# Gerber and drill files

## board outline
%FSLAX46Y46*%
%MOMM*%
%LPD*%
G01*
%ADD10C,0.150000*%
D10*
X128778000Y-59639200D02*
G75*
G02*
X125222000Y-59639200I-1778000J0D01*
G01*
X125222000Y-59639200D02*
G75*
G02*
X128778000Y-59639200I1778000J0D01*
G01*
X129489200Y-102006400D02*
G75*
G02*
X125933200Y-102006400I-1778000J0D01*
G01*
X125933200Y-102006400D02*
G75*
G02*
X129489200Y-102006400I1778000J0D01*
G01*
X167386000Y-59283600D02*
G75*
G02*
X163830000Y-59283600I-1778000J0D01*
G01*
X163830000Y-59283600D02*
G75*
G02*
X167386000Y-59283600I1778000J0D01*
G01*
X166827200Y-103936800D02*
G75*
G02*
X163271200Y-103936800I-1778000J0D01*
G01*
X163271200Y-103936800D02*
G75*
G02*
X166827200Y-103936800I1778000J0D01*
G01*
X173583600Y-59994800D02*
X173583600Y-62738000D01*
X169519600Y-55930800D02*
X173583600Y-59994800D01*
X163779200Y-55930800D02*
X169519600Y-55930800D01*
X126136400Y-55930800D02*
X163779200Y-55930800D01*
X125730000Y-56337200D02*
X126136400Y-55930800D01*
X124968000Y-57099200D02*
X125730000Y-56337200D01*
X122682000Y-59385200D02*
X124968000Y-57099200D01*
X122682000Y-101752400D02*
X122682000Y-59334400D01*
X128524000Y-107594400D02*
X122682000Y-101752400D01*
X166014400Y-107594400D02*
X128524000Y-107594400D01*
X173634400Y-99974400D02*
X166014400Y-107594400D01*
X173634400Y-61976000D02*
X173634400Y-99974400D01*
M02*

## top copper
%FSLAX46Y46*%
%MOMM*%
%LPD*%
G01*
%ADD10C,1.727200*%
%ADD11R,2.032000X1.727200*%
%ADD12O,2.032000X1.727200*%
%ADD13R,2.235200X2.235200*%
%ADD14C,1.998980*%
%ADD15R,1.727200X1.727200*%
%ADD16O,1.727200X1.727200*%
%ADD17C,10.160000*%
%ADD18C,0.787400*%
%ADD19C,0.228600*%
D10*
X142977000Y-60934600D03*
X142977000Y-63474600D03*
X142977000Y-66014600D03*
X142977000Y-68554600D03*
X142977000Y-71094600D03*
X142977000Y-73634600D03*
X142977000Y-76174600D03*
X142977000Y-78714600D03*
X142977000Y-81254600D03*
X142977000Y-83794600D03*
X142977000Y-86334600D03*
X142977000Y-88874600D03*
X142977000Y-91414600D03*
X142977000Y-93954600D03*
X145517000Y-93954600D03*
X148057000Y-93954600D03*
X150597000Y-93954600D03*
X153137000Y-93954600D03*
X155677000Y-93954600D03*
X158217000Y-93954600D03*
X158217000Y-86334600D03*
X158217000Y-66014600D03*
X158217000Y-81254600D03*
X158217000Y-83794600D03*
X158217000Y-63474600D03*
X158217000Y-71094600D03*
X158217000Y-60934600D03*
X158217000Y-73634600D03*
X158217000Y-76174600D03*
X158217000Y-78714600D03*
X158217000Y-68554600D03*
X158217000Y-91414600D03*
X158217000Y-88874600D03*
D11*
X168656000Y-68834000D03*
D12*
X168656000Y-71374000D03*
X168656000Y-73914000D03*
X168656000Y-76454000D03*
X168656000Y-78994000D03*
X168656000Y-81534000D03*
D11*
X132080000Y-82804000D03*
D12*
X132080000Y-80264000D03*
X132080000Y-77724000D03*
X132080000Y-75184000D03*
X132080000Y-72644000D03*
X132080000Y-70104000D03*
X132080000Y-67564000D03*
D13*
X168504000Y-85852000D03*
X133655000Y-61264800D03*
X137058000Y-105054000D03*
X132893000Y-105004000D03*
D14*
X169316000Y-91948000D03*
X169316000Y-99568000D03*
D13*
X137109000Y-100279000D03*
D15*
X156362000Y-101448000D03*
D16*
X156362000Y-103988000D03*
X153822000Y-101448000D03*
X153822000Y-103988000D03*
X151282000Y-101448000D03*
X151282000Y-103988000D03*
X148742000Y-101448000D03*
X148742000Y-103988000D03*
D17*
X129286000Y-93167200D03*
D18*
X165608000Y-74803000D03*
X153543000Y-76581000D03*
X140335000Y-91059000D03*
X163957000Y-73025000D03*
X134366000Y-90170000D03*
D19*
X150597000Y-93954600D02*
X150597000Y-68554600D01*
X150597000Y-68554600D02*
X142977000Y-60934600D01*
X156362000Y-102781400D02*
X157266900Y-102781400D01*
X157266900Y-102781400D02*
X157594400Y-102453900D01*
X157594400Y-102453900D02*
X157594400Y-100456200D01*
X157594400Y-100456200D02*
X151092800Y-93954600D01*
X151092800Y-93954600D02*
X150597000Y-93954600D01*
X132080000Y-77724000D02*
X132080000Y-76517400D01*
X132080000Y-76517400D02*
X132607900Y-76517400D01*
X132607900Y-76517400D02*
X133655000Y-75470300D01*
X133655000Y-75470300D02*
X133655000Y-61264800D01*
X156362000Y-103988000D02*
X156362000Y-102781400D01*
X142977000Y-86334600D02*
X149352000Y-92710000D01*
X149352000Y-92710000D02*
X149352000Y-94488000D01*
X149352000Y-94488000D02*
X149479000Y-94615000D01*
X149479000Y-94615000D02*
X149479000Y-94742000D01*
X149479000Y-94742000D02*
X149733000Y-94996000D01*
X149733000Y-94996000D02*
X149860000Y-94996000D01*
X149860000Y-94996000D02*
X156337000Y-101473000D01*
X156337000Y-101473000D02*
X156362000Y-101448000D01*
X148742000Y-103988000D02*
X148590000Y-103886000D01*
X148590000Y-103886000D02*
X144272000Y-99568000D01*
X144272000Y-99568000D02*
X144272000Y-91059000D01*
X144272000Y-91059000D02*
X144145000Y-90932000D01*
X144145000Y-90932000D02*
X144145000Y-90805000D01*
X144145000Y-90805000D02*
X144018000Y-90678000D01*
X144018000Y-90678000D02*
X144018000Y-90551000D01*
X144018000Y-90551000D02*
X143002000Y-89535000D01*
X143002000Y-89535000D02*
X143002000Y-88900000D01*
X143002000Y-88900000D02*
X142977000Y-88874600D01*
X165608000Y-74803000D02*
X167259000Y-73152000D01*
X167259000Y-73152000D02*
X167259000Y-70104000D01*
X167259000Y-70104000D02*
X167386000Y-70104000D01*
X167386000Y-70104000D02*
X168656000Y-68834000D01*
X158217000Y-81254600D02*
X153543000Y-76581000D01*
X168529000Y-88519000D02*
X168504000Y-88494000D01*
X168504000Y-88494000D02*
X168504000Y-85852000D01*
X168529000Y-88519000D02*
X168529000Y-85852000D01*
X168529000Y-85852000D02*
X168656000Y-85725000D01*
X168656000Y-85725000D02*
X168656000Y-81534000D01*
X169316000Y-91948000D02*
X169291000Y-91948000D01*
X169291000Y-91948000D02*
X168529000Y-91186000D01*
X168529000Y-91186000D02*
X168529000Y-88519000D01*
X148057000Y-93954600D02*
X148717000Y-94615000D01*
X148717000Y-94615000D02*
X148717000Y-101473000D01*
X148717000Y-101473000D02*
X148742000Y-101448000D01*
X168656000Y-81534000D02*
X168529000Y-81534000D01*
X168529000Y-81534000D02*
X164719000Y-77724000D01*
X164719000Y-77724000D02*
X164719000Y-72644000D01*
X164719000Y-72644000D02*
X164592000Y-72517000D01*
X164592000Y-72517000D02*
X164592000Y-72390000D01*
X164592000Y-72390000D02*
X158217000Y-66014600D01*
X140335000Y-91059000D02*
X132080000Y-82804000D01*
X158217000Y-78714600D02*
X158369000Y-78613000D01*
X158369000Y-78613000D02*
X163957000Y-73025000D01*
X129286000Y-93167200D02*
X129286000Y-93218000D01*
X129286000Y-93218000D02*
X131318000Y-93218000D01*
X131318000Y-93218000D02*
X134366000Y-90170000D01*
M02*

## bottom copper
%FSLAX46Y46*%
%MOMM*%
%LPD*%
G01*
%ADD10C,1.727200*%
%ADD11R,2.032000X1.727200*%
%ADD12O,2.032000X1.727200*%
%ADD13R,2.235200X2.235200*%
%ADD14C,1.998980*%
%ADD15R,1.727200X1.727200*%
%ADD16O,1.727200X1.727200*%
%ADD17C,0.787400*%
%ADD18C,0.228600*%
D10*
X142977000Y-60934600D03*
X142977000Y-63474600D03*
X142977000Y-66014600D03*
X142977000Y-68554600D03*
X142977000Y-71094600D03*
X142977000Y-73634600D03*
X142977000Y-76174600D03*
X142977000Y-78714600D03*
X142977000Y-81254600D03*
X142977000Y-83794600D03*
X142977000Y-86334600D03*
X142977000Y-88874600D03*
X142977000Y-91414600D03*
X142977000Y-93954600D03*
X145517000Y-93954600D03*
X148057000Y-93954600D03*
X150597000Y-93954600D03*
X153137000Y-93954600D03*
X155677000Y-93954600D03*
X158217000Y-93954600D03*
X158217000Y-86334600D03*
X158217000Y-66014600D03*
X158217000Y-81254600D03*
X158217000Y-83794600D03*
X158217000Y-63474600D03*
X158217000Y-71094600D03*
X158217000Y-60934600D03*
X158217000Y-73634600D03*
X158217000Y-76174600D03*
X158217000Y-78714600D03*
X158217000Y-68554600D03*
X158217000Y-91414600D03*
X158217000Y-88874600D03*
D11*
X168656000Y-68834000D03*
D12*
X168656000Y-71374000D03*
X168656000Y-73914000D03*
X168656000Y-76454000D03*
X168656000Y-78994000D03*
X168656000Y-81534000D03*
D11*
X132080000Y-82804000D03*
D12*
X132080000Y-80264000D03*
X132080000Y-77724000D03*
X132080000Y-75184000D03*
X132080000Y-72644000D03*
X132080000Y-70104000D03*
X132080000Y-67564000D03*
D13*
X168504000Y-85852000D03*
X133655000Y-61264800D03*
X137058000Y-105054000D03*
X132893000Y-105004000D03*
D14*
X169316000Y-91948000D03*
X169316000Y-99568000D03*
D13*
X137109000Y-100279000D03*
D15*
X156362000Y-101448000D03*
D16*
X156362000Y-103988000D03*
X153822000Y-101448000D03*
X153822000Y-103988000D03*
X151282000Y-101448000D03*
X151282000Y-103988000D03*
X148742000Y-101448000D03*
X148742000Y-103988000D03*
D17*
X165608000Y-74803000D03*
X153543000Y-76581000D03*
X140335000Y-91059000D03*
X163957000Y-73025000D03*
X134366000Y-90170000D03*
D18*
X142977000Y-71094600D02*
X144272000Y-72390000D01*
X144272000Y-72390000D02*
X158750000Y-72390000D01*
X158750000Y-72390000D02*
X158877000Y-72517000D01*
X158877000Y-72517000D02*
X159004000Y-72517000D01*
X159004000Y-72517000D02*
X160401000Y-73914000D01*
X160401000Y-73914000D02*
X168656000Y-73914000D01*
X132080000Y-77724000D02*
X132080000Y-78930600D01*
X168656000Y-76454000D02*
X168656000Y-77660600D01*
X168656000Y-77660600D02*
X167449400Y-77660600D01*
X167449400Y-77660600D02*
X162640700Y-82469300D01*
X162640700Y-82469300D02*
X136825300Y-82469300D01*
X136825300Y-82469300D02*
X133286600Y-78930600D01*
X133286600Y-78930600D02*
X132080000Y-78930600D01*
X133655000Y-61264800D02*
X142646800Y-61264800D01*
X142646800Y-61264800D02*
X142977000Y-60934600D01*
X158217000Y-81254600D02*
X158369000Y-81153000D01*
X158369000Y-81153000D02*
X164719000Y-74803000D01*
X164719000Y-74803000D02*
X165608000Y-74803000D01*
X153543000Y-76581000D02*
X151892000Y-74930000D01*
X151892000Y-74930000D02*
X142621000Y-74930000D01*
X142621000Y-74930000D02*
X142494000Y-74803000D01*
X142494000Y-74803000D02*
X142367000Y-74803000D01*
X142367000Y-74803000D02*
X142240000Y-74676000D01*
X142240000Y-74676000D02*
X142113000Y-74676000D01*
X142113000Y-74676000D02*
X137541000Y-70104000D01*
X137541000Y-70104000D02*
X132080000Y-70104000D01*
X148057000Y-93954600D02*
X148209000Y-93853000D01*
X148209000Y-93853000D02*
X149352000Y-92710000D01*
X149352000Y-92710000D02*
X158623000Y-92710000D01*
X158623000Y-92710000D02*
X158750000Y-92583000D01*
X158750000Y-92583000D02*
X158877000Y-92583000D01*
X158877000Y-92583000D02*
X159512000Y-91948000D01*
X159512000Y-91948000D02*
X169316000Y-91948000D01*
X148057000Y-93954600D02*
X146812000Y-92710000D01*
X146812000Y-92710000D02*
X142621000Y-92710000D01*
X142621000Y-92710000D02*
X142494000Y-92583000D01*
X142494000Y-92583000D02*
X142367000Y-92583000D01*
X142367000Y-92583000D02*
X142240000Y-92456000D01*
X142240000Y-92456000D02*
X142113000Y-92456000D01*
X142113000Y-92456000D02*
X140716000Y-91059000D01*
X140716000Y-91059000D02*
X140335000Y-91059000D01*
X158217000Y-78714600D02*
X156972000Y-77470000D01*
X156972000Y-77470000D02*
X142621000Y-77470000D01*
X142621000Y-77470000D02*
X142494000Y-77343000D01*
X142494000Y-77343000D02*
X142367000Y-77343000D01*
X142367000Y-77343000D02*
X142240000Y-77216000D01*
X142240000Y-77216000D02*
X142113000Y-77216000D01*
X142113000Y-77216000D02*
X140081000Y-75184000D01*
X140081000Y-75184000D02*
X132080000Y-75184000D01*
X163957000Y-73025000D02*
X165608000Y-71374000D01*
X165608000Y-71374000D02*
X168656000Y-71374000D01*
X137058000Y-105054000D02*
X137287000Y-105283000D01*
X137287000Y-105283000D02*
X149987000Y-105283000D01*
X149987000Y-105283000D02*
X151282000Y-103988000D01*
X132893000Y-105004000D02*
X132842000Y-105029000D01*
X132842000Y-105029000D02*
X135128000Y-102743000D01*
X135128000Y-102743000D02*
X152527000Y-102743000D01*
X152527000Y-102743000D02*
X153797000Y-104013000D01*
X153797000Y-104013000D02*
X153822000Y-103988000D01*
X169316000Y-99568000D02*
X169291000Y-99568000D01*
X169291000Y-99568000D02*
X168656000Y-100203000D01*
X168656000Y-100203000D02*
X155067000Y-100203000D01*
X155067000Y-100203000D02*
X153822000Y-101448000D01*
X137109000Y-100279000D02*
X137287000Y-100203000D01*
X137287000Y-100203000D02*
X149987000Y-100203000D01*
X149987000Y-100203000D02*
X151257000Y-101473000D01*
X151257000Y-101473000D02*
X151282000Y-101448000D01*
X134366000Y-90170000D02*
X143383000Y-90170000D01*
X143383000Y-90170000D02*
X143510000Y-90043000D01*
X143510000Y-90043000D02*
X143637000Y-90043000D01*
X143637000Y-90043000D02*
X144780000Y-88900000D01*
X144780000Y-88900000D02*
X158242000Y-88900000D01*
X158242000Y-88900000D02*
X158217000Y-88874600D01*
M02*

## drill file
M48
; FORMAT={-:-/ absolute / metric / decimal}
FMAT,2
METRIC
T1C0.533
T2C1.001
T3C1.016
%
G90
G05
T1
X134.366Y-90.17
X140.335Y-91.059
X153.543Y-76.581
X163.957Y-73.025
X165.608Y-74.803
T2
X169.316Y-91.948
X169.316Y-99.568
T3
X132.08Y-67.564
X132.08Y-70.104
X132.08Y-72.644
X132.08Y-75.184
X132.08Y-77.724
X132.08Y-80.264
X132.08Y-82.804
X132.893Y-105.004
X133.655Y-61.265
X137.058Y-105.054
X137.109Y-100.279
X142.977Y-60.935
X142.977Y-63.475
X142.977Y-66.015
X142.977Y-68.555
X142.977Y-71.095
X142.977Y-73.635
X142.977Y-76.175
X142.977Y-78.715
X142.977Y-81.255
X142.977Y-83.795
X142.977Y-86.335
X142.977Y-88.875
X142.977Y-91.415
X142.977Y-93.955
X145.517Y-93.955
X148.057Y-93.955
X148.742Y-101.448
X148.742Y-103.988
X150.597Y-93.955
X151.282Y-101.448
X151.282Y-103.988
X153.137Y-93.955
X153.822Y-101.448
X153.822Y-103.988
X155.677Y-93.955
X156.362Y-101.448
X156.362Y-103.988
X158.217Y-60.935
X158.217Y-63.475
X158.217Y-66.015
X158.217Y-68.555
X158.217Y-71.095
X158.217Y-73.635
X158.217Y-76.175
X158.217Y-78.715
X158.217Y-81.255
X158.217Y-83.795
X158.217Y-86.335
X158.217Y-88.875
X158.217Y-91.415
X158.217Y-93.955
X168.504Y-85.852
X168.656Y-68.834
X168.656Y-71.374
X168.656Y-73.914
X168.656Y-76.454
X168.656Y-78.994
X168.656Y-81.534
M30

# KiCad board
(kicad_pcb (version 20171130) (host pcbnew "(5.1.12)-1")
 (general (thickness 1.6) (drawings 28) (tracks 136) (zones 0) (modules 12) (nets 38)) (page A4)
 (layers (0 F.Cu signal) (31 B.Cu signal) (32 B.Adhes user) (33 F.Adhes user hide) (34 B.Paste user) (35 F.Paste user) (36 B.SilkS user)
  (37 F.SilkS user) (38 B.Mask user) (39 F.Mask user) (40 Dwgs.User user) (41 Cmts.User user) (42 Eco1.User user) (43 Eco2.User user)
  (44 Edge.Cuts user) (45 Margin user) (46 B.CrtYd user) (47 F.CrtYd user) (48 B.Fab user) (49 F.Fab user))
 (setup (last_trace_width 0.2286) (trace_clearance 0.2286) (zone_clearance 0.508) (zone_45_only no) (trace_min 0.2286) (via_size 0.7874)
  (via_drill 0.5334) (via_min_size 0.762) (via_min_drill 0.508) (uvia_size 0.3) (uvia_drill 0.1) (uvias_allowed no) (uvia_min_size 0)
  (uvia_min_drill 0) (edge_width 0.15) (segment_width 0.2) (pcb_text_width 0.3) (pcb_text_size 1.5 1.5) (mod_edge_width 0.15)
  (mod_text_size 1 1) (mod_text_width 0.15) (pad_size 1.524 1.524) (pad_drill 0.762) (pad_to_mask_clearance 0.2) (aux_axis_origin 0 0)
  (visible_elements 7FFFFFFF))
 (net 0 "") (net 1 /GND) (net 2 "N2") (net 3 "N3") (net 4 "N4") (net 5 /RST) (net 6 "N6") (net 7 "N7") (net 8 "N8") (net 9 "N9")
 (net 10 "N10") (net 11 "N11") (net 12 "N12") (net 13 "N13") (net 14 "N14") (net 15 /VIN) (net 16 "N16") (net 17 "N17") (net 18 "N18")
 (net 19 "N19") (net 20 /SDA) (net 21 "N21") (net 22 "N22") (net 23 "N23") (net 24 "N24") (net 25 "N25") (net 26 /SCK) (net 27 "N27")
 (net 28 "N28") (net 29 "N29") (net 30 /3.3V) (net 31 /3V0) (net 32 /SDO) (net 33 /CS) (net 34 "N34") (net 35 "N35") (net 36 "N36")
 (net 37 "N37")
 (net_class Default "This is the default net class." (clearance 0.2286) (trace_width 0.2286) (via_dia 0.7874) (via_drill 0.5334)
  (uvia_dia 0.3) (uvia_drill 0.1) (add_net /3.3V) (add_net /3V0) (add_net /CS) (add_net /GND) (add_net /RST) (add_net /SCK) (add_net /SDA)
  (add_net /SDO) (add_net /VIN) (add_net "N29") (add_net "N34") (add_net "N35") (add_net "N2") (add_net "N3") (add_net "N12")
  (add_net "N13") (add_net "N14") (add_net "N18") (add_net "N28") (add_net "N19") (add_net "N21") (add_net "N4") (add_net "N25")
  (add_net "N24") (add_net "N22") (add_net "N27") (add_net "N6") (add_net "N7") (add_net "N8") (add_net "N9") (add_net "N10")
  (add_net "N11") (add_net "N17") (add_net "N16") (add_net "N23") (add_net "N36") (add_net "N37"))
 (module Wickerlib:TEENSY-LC (layer F.Cu) (at 153.137 71.0946)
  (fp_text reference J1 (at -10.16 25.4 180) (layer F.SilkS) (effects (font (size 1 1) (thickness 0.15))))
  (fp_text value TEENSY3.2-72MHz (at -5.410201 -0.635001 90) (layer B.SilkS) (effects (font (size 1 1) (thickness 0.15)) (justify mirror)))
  (pad G1 thru_hole circle (at -10.16 -10.16) (size 1.7272 1.7272) (drill 1.016) (layers *.Cu *.Mask F.SilkS) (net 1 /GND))
  (pad 0 thru_hole circle (at -10.16 -7.62) (size 1.7272 1.7272) (drill 1.016) (layers *.Cu *.Mask F.SilkS) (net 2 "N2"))
  (pad 1 thru_hole circle (at -10.16 -5.08) (size 1.7272 1.7272) (drill 1.016) (layers *.Cu *.Mask F.SilkS) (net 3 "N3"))
  (pad 2 thru_hole circle (at -10.16 -2.54) (size 1.7272 1.7272) (drill 1.016) (layers *.Cu *.Mask F.SilkS) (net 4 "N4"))
  (pad 3 thru_hole circle (at -10.16 0) (size 1.7272 1.7272) (drill 1.016) (layers *.Cu *.Mask F.SilkS) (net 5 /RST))
  (pad 4 thru_hole circle (at -10.16 2.54) (size 1.7272 1.7272) (drill 1.016) (layers *.Cu *.Mask F.SilkS) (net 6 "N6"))
  (pad 5 thru_hole circle (at -10.16 5.08) (size 1.7272 1.7272) (drill 1.016) (layers *.Cu *.Mask F.SilkS) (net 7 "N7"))
  (pad 6 thru_hole circle (at -10.16 7.62) (size 1.7272 1.7272) (drill 1.016) (layers *.Cu *.Mask F.SilkS) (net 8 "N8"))
  (pad 7 thru_hole circle (at -10.16 10.16) (size 1.7272 1.7272) (drill 1.016) (layers *.Cu *.Mask F.SilkS) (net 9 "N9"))
  (pad 8 thru_hole circle (at -10.16 12.7) (size 1.7272 1.7272) (drill 1.016) (layers *.Cu *.Mask F.SilkS) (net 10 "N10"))
  (pad 9 thru_hole circle (at -10.16 15.24) (size 1.7272 1.7272) (drill 1.016) (layers *.Cu *.Mask F.SilkS) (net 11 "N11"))
  (pad 10 thru_hole circle (at -10.16 17.78) (size 1.7272 1.7272) (drill 1.016) (layers *.Cu *.Mask F.SilkS) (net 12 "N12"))
  (pad 11 thru_hole circle (at -10.16 20.32) (size 1.7272 1.7272) (drill 1.016) (layers *.Cu *.Mask F.SilkS) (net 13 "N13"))
  (pad 12 thru_hole circle (at -10.16 22.86) (size 1.7272 1.7272) (drill 1.016) (layers *.Cu *.Mask F.SilkS) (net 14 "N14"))
  (pad 17A thru_hole circle (at -7.62 22.86) (size 1.7272 1.7272) (drill 1.016) (layers *.Cu *.Mask F.SilkS))
  (pad 3V1 thru_hole circle (at -5.08 22.86) (size 1.7272 1.7272) (drill 1.016) (layers *.Cu *.Mask F.SilkS) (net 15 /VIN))
  (pad G2 thru_hole circle (at -2.54 22.86) (size 1.7272 1.7272) (drill 1.016) (layers *.Cu *.Mask F.SilkS) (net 1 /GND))
  (pad PGM thru_hole circle (at 0 22.86) (size 1.7272 1.7272) (drill 1.016) (layers *.Cu *.Mask F.SilkS) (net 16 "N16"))
  (pad DAC thru_hole circle (at 2.54 22.86) (size 1.7272 1.7272) (drill 1.016) (layers *.Cu *.Mask F.SilkS) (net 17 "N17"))
  (pad 13 thru_hole circle (at 5.08 22.86) (size 1.7272 1.7272) (drill 1.016) (layers *.Cu *.Mask F.SilkS) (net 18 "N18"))
  (pad 16 thru_hole circle (at 5.08 15.24) (size 1.7272 1.7272) (drill 1.016) (layers *.Cu *.Mask F.SilkS) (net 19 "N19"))
  (pad 3V2 thru_hole circle (at 5.08 -5.08) (size 1.7272 1.7272) (drill 1.016) (layers *.Cu *.Mask F.SilkS) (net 15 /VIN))
  (pad 18 thru_hole circle (at 5.08 10.16) (size 1.7272 1.7272) (drill 1.016) (layers *.Cu *.Mask F.SilkS) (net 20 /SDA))
  (pad 17 thru_hole circle (at 5.08 12.7) (size 1.7272 1.7272) (drill 1.016) (layers *.Cu *.Mask F.SilkS) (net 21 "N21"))
  (pad G3 thru_hole circle (at 5.08 -7.62) (size 1.7272 1.7272) (drill 1.016) (layers *.Cu *.Mask F.SilkS))
  (pad 22 thru_hole circle (at 5.08 0) (size 1.7272 1.7272) (drill 1.016) (layers *.Cu *.Mask F.SilkS) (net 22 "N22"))
  (pad VIN thru_hole circle (at 5.08 -10.16) (size 1.7272 1.7272) (drill 1.016) (layers *.Cu *.Mask F.SilkS) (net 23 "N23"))
  (pad 21 thru_hole circle (at 5.08 2.54) (size 1.7272 1.7272) (drill 1.016) (layers *.Cu *.Mask F.SilkS) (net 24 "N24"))
  (pad 20 thru_hole circle (at 5.08 5.08) (size 1.7272 1.7272) (drill 1.016) (layers *.Cu *.Mask F.SilkS) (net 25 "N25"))
  (pad 19 thru_hole circle (at 5.08 7.62) (size 1.7272 1.7272) (drill 1.016) (layers *.Cu *.Mask F.SilkS) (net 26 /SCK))
  (pad 23 thru_hole circle (at 5.08 -2.54) (size 1.7272 1.7272) (drill 1.016) (layers *.Cu *.Mask F.SilkS) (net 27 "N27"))
  (pad 14 thru_hole circle (at 5.08 20.32) (size 1.7272 1.7272) (drill 1.016) (layers *.Cu *.Mask F.SilkS) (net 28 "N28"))
  (pad 15 thru_hole circle (at 5.08 17.78) (size 1.7272 1.7272) (drill 1.016) (layers *.Cu *.Mask F.SilkS) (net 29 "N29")))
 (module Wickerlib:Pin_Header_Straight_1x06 (layer F.Cu) (at 168.656 68.834)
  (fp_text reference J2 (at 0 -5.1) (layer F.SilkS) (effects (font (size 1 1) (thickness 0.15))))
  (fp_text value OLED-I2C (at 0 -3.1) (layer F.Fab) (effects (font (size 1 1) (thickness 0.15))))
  (pad 1 thru_hole rect (at 0 0) (size 2.032 1.7272) (drill 1.016) (layers *.Cu *.Mask F.SilkS) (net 20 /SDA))
  (pad 2 thru_hole oval (at 0 2.54) (size 2.032 1.7272) (drill 1.016) (layers *.Cu *.Mask F.SilkS) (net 26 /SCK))
  (pad 3 thru_hole oval (at 0 5.08) (size 2.032 1.7272) (drill 1.016) (layers *.Cu *.Mask F.SilkS) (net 5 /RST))
  (pad 4 thru_hole oval (at 0 7.62) (size 2.032 1.7272) (drill 1.016) (layers *.Cu *.Mask F.SilkS) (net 1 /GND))
  (pad 5 thru_hole oval (at 0 10.16) (size 2.032 1.7272) (drill 1.016) (layers *.Cu *.Mask F.SilkS) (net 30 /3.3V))
  (pad 6 thru_hole oval (at 0 12.7) (size 2.032 1.7272) (drill 1.016) (layers *.Cu *.Mask F.SilkS) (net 15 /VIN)))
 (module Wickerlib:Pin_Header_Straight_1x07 (layer F.Cu) (at 132.08 82.804 180)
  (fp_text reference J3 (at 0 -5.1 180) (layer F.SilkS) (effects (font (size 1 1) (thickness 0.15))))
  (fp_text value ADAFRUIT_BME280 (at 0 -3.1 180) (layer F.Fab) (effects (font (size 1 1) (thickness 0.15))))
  (pad 1 thru_hole rect (at 0 0 180) (size 2.032 1.7272) (drill 1.016) (layers *.Cu *.Mask F.SilkS) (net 15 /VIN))
  (pad 2 thru_hole oval (at 0 2.54 180) (size 2.032 1.7272) (drill 1.016) (layers *.Cu *.Mask F.SilkS) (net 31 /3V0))
  (pad 3 thru_hole oval (at 0 5.08 180) (size 2.032 1.7272) (drill 1.016) (layers *.Cu *.Mask F.SilkS) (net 1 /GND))
  (pad 4 thru_hole oval (at 0 7.62 180) (size 2.032 1.7272) (drill 1.016) (layers *.Cu *.Mask F.SilkS) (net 26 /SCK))
  (pad 5 thru_hole oval (at 0 10.16 180) (size 2.032 1.7272) (drill 1.016) (layers *.Cu *.Mask F.SilkS) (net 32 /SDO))
  (pad 6 thru_hole oval (at 0 12.7 180) (size 2.032 1.7272) (drill 1.016) (layers *.Cu *.Mask F.SilkS) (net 20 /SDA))
  (pad 7 thru_hole oval (at 0 15.24 180) (size 2.032 1.7272) (drill 1.016) (layers *.Cu *.Mask F.SilkS) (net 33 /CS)))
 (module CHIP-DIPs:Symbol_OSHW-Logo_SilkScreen (layer F.Cu) (at 129.286 93.0148 270)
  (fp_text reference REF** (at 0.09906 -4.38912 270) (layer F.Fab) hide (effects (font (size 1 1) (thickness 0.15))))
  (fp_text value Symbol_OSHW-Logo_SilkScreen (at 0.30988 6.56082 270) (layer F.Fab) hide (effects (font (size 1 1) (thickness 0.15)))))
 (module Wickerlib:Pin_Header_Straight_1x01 (layer F.Cu) (at 168.504 85.852 90)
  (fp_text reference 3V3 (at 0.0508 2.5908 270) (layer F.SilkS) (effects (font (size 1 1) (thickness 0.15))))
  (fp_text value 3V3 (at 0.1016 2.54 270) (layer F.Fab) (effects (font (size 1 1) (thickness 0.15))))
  (pad 1 thru_hole rect (at 0 0 90) (size 2.2352 2.2352) (drill 1.016) (layers *.Cu *.Mask F.SilkS) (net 15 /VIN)))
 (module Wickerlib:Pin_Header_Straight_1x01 (layer F.Cu) (at 133.655 61.2648)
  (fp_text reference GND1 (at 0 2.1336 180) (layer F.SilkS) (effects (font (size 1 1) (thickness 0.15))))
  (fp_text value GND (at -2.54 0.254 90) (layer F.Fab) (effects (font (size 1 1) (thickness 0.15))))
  (pad 1 thru_hole rect (at 0 0) (size 2.2352 2.2352) (drill 1.016) (layers *.Cu *.Mask F.SilkS) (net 1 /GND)))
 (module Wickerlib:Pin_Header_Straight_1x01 (layer F.Cu) (at 137.058 105.054 270)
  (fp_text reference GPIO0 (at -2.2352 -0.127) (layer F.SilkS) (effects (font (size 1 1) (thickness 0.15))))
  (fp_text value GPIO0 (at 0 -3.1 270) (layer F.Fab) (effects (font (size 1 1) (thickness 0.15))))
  (pad 1 thru_hole rect (at 0 0 270) (size 2.2352 2.2352) (drill 1.016) (layers *.Cu *.Mask F.SilkS) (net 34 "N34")))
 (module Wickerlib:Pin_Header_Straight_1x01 (layer F.Cu) (at 132.893 105.004 270)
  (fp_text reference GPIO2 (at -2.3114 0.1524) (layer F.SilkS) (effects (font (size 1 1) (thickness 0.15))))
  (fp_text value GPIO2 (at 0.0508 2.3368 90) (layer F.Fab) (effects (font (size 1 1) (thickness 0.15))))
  (pad 1 thru_hole rect (at 0 0 270) (size 2.2352 2.2352) (drill 1.016) (layers *.Cu *.Mask F.SilkS) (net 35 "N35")))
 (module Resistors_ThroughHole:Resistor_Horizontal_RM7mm (layer F.Cu) (at 169.316 91.948 270)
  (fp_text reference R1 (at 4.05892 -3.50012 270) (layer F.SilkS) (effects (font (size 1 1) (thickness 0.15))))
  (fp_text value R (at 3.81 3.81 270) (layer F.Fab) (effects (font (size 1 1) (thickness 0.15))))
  (pad 1 thru_hole circle (at 0 0 270) (size 1.99898 1.99898) (drill 1.00076) (layers *.Cu *.SilkS *.Mask) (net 15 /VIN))
  (pad 2 thru_hole circle (at 7.62 0 270) (size 1.99898 1.99898) (drill 1.00076) (layers *.Cu *.SilkS *.Mask) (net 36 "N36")))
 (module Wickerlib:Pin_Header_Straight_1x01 (layer F.Cu) (at 137.109 100.279 270)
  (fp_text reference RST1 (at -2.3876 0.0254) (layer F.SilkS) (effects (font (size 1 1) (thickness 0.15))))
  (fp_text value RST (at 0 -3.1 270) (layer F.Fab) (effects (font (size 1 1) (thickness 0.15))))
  (pad 1 thru_hole rect (at 0 0 270) (size 2.2352 2.2352) (drill 1.016) (layers *.Cu *.Mask F.SilkS) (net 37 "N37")))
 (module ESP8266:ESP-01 (layer F.Cu) (at 156.362 101.448 270)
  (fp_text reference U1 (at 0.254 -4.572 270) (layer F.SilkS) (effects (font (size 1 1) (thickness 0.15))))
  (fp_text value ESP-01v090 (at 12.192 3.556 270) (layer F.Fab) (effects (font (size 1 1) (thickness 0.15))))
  (pad 1 thru_hole rect (at 0 0 270) (size 1.7272 1.7272) (drill 1.016) (layers *.Cu *.Mask F.SilkS) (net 11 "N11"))
  (pad 2 thru_hole oval (at 2.54 0 270) (size 1.7272 1.7272) (drill 1.016) (layers *.Cu *.Mask F.SilkS) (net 1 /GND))
  (pad 3 thru_hole oval (at 0 2.54 270) (size 1.7272 1.7272) (drill 1.016) (layers *.Cu *.Mask F.SilkS) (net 36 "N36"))
  (pad 4 thru_hole oval (at 2.54 2.54 270) (size 1.7272 1.7272) (drill 1.016) (layers *.Cu *.Mask F.SilkS) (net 35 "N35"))
  (pad 5 thru_hole oval (at 0 5.08 270) (size 1.7272 1.7272) (drill 1.016) (layers *.Cu *.Mask F.SilkS) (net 37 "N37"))
  (pad 6 thru_hole oval (at 2.54 5.08 270) (size 1.7272 1.7272) (drill 1.016) (layers *.Cu *.Mask F.SilkS) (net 34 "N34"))
  (pad 7 thru_hole oval (at 0 7.62 270) (size 1.7272 1.7272) (drill 1.016) (layers *.Cu *.Mask F.SilkS) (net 15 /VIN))
  (pad 8 thru_hole oval (at 2.54 7.62 270) (size 1.7272 1.7272) (drill 1.016) (layers *.Cu *.Mask F.SilkS) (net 12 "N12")))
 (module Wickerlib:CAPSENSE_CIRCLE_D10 (layer F.Cu) (at 129.286 93.1672)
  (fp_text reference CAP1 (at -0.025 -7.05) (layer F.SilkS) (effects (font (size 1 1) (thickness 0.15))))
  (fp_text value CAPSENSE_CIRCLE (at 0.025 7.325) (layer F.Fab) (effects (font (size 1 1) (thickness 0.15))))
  (pad 1 smd circle (at 0 0) (size 10.16 10.16) (layers F.Cu) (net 29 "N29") (clearance 0.508)))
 (gr_circle (center 127 59.6392) (end 128.4224 60.706) (layer Edge.Cuts) (width 0.15))
 (gr_circle (center 127.7112 102.0064) (end 129.1336 103.0732) (layer Edge.Cuts) (width 0.15))
 (gr_circle (center 165.608 59.2836) (end 167.0304 60.3504) (layer Edge.Cuts) (width 0.15))
 (gr_circle (center 165.0492 103.9368) (end 166.4716 105.0036) (layer Edge.Cuts) (width 0.15))
 (gr_line (start 173.5836 59.9948) (end 173.5836 62.738) (angle 90) (layer Edge.Cuts) (width 0.15))
 (gr_line (start 169.5196 55.9308) (end 173.5836 59.9948) (angle 90) (layer Edge.Cuts) (width 0.15))
 (gr_line (start 163.7792 55.9308) (end 169.5196 55.9308) (angle 90) (layer Edge.Cuts) (width 0.15))
 (gr_line (start 126.1364 55.9308) (end 163.7792 55.9308) (angle 90) (layer Edge.Cuts) (width 0.15))
 (gr_line (start 125.73 56.3372) (end 126.1364 55.9308) (angle 90) (layer Edge.Cuts) (width 0.15))
 (gr_line (start 124.968 57.0992) (end 125.73 56.3372) (angle 90) (layer Edge.Cuts) (width 0.15))
 (gr_line (start 122.682 59.3852) (end 124.968 57.0992) (angle 90) (layer Edge.Cuts) (width 0.15))
 (gr_line (start 122.682 101.7524) (end 122.682 59.3344) (angle 90) (layer Edge.Cuts) (width 0.15))
 (gr_line (start 128.524 107.5944) (end 122.682 101.7524) (angle 90) (layer Edge.Cuts) (width 0.15))
 (gr_line (start 166.0144 107.5944) (end 128.524 107.5944) (angle 90) (layer Edge.Cuts) (width 0.15))
 (gr_line (start 173.6344 99.9744) (end 166.0144 107.5944) (angle 90) (layer Edge.Cuts) (width 0.15))
 (gr_line (start 173.6344 61.976) (end 173.6344 99.9744) (angle 90) (layer Edge.Cuts) (width 0.15))
 (segment (start 142.977 71.0946) (end 144.272 72.39) (width 0.2286) (layer B.Cu) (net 5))
 (segment (start 144.272 72.39) (end 158.75 72.39) (width 0.2286) (layer B.Cu) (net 5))
 (segment (start 158.75 72.39) (end 158.877 72.517) (width 0.2286) (layer B.Cu) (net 5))
 (segment (start 158.877 72.517) (end 159.004 72.517) (width 0.2286) (layer B.Cu) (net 5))
 (segment (start 159.004 72.517) (end 160.401 73.914) (width 0.2286) (layer B.Cu) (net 5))
 (segment (start 160.401 73.914) (end 168.656 73.914) (width 0.2286) (layer B.Cu) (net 5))
 (segment (start 150.597 93.9546) (end 150.597 68.5546) (width 0.2286) (layer F.Cu) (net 1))
 (segment (start 150.597 68.5546) (end 142.977 60.9346) (width 0.2286) (layer F.Cu) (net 1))
 (segment (start 156.362 102.7814) (end 157.2669 102.7814) (width 0.2286) (layer F.Cu) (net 1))
 (segment (start 157.2669 102.7814) (end 157.5944 102.4539) (width 0.2286) (layer F.Cu) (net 1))
 (segment (start 157.5944 102.4539) (end 157.5944 100.4562) (width 0.2286) (layer F.Cu) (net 1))
 (segment (start 157.5944 100.4562) (end 151.0928 93.9546) (width 0.2286) (layer F.Cu) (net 1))
 (segment (start 151.0928 93.9546) (end 150.597 93.9546) (width 0.2286) (layer F.Cu) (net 1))
 (segment (start 132.08 77.724) (end 132.08 78.9306) (width 0.2286) (layer B.Cu) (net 1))
 (segment (start 168.656 76.454) (end 168.656 77.6606) (width 0.2286) (layer B.Cu) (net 1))
 (segment (start 168.656 77.6606) (end 167.4494 77.6606) (width 0.2286) (layer B.Cu) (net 1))
 (segment (start 167.4494 77.6606) (end 162.6407 82.4693) (width 0.2286) (layer B.Cu) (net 1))
 (segment (start 162.6407 82.4693) (end 136.8253 82.4693) (width 0.2286) (layer B.Cu) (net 1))
 (segment (start 136.8253 82.4693) (end 133.2866 78.9306) (width 0.2286) (layer B.Cu) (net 1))
 (segment (start 133.2866 78.9306) (end 132.08 78.9306) (width 0.2286) (layer B.Cu) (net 1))
 (segment (start 132.08 77.724) (end 132.08 76.5174) (width 0.2286) (layer F.Cu) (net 1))
 (segment (start 132.08 76.5174) (end 132.6079 76.5174) (width 0.2286) (layer F.Cu) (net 1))
 (segment (start 132.6079 76.5174) (end 133.655 75.4703) (width 0.2286) (layer F.Cu) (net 1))
 (segment (start 133.655 75.4703) (end 133.655 61.2648) (width 0.2286) (layer F.Cu) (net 1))
 (segment (start 133.655 61.2648) (end 142.6468 61.2648) (width 0.2286) (layer B.Cu) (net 1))
 (segment (start 142.6468 61.2648) (end 142.977 60.9346) (width 0.2286) (layer B.Cu) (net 1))
 (segment (start 156.362 103.988) (end 156.362 102.7814) (width 0.2286) (layer F.Cu) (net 1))
 (segment (start 142.977 86.3346) (end 149.352 92.71) (width 0.2286) (layer F.Cu) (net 11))
 (segment (start 149.352 92.71) (end 149.352 94.488) (width 0.2286) (layer F.Cu) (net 11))
 (segment (start 149.352 94.488) (end 149.479 94.615) (width 0.2286) (layer F.Cu) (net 11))
 (segment (start 149.479 94.615) (end 149.479 94.742) (width 0.2286) (layer F.Cu) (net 11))
 (segment (start 149.479 94.742) (end 149.733 94.996) (width 0.2286) (layer F.Cu) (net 11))
 (segment (start 149.733 94.996) (end 149.86 94.996) (width 0.2286) (layer F.Cu) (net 11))
 (segment (start 149.86 94.996) (end 156.337 101.473) (width 0.2286) (layer F.Cu) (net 11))
 (segment (start 156.337 101.473) (end 156.362 101.448) (width 0.2286) (layer F.Cu) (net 11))
 (segment (start 148.742 103.988) (end 148.59 103.886) (width 0.2286) (layer F.Cu) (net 12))
 (segment (start 148.59 103.886) (end 144.272 99.568) (width 0.2286) (layer F.Cu) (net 12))
 (segment (start 144.272 99.568) (end 144.272 91.059) (width 0.2286) (layer F.Cu) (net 12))
 (segment (start 144.272 91.059) (end 144.145 90.932) (width 0.2286) (layer F.Cu) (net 12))
 (segment (start 144.145 90.932) (end 144.145 90.805) (width 0.2286) (layer F.Cu) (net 12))
 (segment (start 144.145 90.805) (end 144.018 90.678) (width 0.2286) (layer F.Cu) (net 12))
 (segment (start 144.018 90.678) (end 144.018 90.551) (width 0.2286) (layer F.Cu) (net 12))
 (segment (start 144.018 90.551) (end 143.002 89.535) (width 0.2286) (layer F.Cu) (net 12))
 (segment (start 143.002 89.535) (end 143.002 88.9) (width 0.2286) (layer F.Cu) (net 12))
 (segment (start 143.002 88.9) (end 142.977 88.8746) (width 0.2286) (layer F.Cu) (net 12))
 (segment (start 165.608 74.803) (end 167.259 73.152) (width 0.2286) (layer F.Cu) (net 20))
 (segment (start 167.259 73.152) (end 167.259 70.104) (width 0.2286) (layer F.Cu) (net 20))
 (segment (start 167.259 70.104) (end 167.386 70.104) (width 0.2286) (layer F.Cu) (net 20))
 (segment (start 167.386 70.104) (end 168.656 68.834) (width 0.2286) (layer F.Cu) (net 20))
 (segment (start 158.217 81.2546) (end 158.369 81.153) (width 0.2286) (layer B.Cu) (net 20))
 (segment (start 158.369 81.153) (end 164.719 74.803) (width 0.2286) (layer B.Cu) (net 20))
 (segment (start 164.719 74.803) (end 165.608 74.803) (width 0.2286) (layer B.Cu) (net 20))
 (segment (start 153.543 76.581) (end 151.892 74.93) (width 0.2286) (layer B.Cu) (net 20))
 (segment (start 151.892 74.93) (end 142.621 74.93) (width 0.2286) (layer B.Cu) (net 20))
 (segment (start 142.621 74.93) (end 142.494 74.803) (width 0.2286) (layer B.Cu) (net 20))
 (segment (start 142.494 74.803) (end 142.367 74.803) (width 0.2286) (layer B.Cu) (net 20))
 (segment (start 142.367 74.803) (end 142.24 74.676) (width 0.2286) (layer B.Cu) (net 20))
 (segment (start 142.24 74.676) (end 142.113 74.676) (width 0.2286) (layer B.Cu) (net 20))
 (segment (start 142.113 74.676) (end 137.541 70.104) (width 0.2286) (layer B.Cu) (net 20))
 (segment (start 137.541 70.104) (end 132.08 70.104) (width 0.2286) (layer B.Cu) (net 20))
 (segment (start 158.217 81.2546) (end 153.543 76.581) (width 0.2286) (layer F.Cu) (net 20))
 (via (at 165.608 74.803) (size 0.7874) (layers F.Cu B.Cu) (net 20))
 (via (at 153.543 76.581) (size 0.7874) (layers F.Cu B.Cu) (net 20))
 (segment (start 168.529 88.519) (end 168.504 88.494) (width 0.2286) (layer F.Cu) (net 15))
 (segment (start 168.504 88.494) (end 168.504 85.852) (width 0.2286) (layer F.Cu) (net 15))
 (segment (start 168.529 88.519) (end 168.529 85.852) (width 0.2286) (layer F.Cu) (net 15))
 (segment (start 168.529 85.852) (end 168.656 85.725) (width 0.2286) (layer F.Cu) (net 15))
 (segment (start 168.656 85.725) (end 168.656 81.534) (width 0.2286) (layer F.Cu) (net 15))
 (segment (start 169.316 91.948) (end 169.291 91.948) (width 0.2286) (layer F.Cu) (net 15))
 (segment (start 169.291 91.948) (end 168.529 91.186) (width 0.2286) (layer F.Cu) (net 15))
 (segment (start 168.529 91.186) (end 168.529 88.519) (width 0.2286) (layer F.Cu) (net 15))
 (segment (start 148.057 93.9546) (end 148.717 94.615) (width 0.2286) (layer F.Cu) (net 15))
 (segment (start 148.717 94.615) (end 148.717 101.473) (width 0.2286) (layer F.Cu) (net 15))
 (segment (start 148.717 101.473) (end 148.742 101.448) (width 0.2286) (layer F.Cu) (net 15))
 (segment (start 148.057 93.9546) (end 148.209 93.853) (width 0.2286) (layer B.Cu) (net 15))
 (segment (start 148.209 93.853) (end 149.352 92.71) (width 0.2286) (layer B.Cu) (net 15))
 (segment (start 149.352 92.71) (end 158.623 92.71) (width 0.2286) (layer B.Cu) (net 15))
 (segment (start 158.623 92.71) (end 158.75 92.583) (width 0.2286) (layer B.Cu) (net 15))
 (segment (start 158.75 92.583) (end 158.877 92.583) (width 0.2286) (layer B.Cu) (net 15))
 (segment (start 158.877 92.583) (end 159.512 91.948) (width 0.2286) (layer B.Cu) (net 15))
 (segment (start 159.512 91.948) (end 169.316 91.948) (width 0.2286) (layer B.Cu) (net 15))
 (segment (start 168.656 81.534) (end 168.529 81.534) (width 0.2286) (layer F.Cu) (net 15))
 (segment (start 168.529 81.534) (end 164.719 77.724) (width 0.2286) (layer F.Cu) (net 15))
 (segment (start 164.719 77.724) (end 164.719 72.644) (width 0.2286) (layer F.Cu) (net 15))
 (segment (start 164.719 72.644) (end 164.592 72.517) (width 0.2286) (layer F.Cu) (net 15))
 (segment (start 164.592 72.517) (end 164.592 72.39) (width 0.2286) (layer F.Cu) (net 15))
 (segment (start 164.592 72.39) (end 158.217 66.0146) (width 0.2286) (layer F.Cu) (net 15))
 (segment (start 140.335 91.059) (end 132.08 82.804) (width 0.2286) (layer F.Cu) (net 15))
 (segment (start 148.057 93.9546) (end 146.812 92.71) (width 0.2286) (layer B.Cu) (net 15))
 (segment (start 146.812 92.71) (end 142.621 92.71) (width 0.2286) (layer B.Cu) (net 15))
 (segment (start 142.621 92.71) (end 142.494 92.583) (width 0.2286) (layer B.Cu) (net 15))
 (segment (start 142.494 92.583) (end 142.367 92.583) (width 0.2286) (layer B.Cu) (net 15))
 (segment (start 142.367 92.583) (end 142.24 92.456) (width 0.2286) (layer B.Cu) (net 15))
 (segment (start 142.24 92.456) (end 142.113 92.456) (width 0.2286) (layer B.Cu) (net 15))
 (segment (start 142.113 92.456) (end 140.716 91.059) (width 0.2286) (layer B.Cu) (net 15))
 (segment (start 140.716 91.059) (end 140.335 91.059) (width 0.2286) (layer B.Cu) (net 15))
 (via (at 140.335 91.059) (size 0.7874) (layers F.Cu B.Cu) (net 15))
 (segment (start 158.217 78.7146) (end 156.972 77.47) (width 0.2286) (layer B.Cu) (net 26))
 (segment (start 156.972 77.47) (end 142.621 77.47) (width 0.2286) (layer B.Cu) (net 26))
 (segment (start 142.621 77.47) (end 142.494 77.343) (width 0.2286) (layer B.Cu) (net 26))
 (segment (start 142.494 77.343) (end 142.367 77.343) (width 0.2286) (layer B.Cu) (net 26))
 (segment (start 142.367 77.343) (end 142.24 77.216) (width 0.2286) (layer B.Cu) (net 26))
 (segment (start 142.24 77.216) (end 142.113 77.216) (width 0.2286) (layer B.Cu) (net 26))
 (segment (start 142.113 77.216) (end 140.081 75.184) (width 0.2286) (layer B.Cu) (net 26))
 (segment (start 140.081 75.184) (end 132.08 75.184) (width 0.2286) (layer B.Cu) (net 26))
 (segment (start 163.957 73.025) (end 165.608 71.374) (width 0.2286) (layer B.Cu) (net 26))
 (segment (start 165.608 71.374) (end 168.656 71.374) (width 0.2286) (layer B.Cu) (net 26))
 (segment (start 158.217 78.7146) (end 158.369 78.613) (width 0.2286) (layer F.Cu) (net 26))
 (segment (start 158.369 78.613) (end 163.957 73.025) (width 0.2286) (layer F.Cu) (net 26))
 (via (at 163.957 73.025) (size 0.7874) (layers F.Cu B.Cu) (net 26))
 (segment (start 137.058 105.054) (end 137.287 105.283) (width 0.2286) (layer B.Cu) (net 34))
 (segment (start 137.287 105.283) (end 149.987 105.283) (width 0.2286) (layer B.Cu) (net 34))
 (segment (start 149.987 105.283) (end 151.282 103.988) (width 0.2286) (layer B.Cu) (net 34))
 (segment (start 132.893 105.004) (end 132.842 105.029) (width 0.2286) (layer B.Cu) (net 35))
 (segment (start 132.842 105.029) (end 135.128 102.743) (width 0.2286) (layer B.Cu) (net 35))
 (segment (start 135.128 102.743) (end 152.527 102.743) (width 0.2286) (layer B.Cu) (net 35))
 (segment (start 152.527 102.743) (end 153.797 104.013) (width 0.2286) (layer B.Cu) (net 35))
 (segment (start 153.797 104.013) (end 153.822 103.988) (width 0.2286) (layer B.Cu) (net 35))
 (segment (start 169.316 99.568) (end 169.291 99.568) (width 0.2286) (layer B.Cu) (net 36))
 (segment (start 169.291 99.568) (end 168.656 100.203) (width 0.2286) (layer B.Cu) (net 36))
 (segment (start 168.656 100.203) (end 155.067 100.203) (width 0.2286) (layer B.Cu) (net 36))
 (segment (start 155.067 100.203) (end 153.822 101.448) (width 0.2286) (layer B.Cu) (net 36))
 (segment (start 137.109 100.279) (end 137.287 100.203) (width 0.2286) (layer B.Cu) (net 37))
 (segment (start 137.287 100.203) (end 149.987 100.203) (width 0.2286) (layer B.Cu) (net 37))
 (segment (start 149.987 100.203) (end 151.257 101.473) (width 0.2286) (layer B.Cu) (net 37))
 (segment (start 151.257 101.473) (end 151.282 101.448) (width 0.2286) (layer B.Cu) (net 37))
 (segment (start 134.366 90.17) (end 143.383 90.17) (width 0.2286) (layer B.Cu) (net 29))
 (segment (start 143.383 90.17) (end 143.51 90.043) (width 0.2286) (layer B.Cu) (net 29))
 (segment (start 143.51 90.043) (end 143.637 90.043) (width 0.2286) (layer B.Cu) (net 29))
 (segment (start 143.637 90.043) (end 144.78 88.9) (width 0.2286) (layer B.Cu) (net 29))
 (segment (start 144.78 88.9) (end 158.242 88.9) (width 0.2286) (layer B.Cu) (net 29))
 (segment (start 158.242 88.9) (end 158.217 88.8746) (width 0.2286) (layer B.Cu) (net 29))
 (segment (start 129.286 93.1672) (end 129.286 93.218) (width 0.2286) (layer F.Cu) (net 29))
 (segment (start 129.286 93.218) (end 131.318 93.218) (width 0.2286) (layer F.Cu) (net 29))
 (segment (start 131.318 93.218) (end 134.366 90.17) (width 0.2286) (layer F.Cu) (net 29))
 (via (at 134.366 90.17) (size 0.7874) (layers F.Cu B.Cu) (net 29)))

